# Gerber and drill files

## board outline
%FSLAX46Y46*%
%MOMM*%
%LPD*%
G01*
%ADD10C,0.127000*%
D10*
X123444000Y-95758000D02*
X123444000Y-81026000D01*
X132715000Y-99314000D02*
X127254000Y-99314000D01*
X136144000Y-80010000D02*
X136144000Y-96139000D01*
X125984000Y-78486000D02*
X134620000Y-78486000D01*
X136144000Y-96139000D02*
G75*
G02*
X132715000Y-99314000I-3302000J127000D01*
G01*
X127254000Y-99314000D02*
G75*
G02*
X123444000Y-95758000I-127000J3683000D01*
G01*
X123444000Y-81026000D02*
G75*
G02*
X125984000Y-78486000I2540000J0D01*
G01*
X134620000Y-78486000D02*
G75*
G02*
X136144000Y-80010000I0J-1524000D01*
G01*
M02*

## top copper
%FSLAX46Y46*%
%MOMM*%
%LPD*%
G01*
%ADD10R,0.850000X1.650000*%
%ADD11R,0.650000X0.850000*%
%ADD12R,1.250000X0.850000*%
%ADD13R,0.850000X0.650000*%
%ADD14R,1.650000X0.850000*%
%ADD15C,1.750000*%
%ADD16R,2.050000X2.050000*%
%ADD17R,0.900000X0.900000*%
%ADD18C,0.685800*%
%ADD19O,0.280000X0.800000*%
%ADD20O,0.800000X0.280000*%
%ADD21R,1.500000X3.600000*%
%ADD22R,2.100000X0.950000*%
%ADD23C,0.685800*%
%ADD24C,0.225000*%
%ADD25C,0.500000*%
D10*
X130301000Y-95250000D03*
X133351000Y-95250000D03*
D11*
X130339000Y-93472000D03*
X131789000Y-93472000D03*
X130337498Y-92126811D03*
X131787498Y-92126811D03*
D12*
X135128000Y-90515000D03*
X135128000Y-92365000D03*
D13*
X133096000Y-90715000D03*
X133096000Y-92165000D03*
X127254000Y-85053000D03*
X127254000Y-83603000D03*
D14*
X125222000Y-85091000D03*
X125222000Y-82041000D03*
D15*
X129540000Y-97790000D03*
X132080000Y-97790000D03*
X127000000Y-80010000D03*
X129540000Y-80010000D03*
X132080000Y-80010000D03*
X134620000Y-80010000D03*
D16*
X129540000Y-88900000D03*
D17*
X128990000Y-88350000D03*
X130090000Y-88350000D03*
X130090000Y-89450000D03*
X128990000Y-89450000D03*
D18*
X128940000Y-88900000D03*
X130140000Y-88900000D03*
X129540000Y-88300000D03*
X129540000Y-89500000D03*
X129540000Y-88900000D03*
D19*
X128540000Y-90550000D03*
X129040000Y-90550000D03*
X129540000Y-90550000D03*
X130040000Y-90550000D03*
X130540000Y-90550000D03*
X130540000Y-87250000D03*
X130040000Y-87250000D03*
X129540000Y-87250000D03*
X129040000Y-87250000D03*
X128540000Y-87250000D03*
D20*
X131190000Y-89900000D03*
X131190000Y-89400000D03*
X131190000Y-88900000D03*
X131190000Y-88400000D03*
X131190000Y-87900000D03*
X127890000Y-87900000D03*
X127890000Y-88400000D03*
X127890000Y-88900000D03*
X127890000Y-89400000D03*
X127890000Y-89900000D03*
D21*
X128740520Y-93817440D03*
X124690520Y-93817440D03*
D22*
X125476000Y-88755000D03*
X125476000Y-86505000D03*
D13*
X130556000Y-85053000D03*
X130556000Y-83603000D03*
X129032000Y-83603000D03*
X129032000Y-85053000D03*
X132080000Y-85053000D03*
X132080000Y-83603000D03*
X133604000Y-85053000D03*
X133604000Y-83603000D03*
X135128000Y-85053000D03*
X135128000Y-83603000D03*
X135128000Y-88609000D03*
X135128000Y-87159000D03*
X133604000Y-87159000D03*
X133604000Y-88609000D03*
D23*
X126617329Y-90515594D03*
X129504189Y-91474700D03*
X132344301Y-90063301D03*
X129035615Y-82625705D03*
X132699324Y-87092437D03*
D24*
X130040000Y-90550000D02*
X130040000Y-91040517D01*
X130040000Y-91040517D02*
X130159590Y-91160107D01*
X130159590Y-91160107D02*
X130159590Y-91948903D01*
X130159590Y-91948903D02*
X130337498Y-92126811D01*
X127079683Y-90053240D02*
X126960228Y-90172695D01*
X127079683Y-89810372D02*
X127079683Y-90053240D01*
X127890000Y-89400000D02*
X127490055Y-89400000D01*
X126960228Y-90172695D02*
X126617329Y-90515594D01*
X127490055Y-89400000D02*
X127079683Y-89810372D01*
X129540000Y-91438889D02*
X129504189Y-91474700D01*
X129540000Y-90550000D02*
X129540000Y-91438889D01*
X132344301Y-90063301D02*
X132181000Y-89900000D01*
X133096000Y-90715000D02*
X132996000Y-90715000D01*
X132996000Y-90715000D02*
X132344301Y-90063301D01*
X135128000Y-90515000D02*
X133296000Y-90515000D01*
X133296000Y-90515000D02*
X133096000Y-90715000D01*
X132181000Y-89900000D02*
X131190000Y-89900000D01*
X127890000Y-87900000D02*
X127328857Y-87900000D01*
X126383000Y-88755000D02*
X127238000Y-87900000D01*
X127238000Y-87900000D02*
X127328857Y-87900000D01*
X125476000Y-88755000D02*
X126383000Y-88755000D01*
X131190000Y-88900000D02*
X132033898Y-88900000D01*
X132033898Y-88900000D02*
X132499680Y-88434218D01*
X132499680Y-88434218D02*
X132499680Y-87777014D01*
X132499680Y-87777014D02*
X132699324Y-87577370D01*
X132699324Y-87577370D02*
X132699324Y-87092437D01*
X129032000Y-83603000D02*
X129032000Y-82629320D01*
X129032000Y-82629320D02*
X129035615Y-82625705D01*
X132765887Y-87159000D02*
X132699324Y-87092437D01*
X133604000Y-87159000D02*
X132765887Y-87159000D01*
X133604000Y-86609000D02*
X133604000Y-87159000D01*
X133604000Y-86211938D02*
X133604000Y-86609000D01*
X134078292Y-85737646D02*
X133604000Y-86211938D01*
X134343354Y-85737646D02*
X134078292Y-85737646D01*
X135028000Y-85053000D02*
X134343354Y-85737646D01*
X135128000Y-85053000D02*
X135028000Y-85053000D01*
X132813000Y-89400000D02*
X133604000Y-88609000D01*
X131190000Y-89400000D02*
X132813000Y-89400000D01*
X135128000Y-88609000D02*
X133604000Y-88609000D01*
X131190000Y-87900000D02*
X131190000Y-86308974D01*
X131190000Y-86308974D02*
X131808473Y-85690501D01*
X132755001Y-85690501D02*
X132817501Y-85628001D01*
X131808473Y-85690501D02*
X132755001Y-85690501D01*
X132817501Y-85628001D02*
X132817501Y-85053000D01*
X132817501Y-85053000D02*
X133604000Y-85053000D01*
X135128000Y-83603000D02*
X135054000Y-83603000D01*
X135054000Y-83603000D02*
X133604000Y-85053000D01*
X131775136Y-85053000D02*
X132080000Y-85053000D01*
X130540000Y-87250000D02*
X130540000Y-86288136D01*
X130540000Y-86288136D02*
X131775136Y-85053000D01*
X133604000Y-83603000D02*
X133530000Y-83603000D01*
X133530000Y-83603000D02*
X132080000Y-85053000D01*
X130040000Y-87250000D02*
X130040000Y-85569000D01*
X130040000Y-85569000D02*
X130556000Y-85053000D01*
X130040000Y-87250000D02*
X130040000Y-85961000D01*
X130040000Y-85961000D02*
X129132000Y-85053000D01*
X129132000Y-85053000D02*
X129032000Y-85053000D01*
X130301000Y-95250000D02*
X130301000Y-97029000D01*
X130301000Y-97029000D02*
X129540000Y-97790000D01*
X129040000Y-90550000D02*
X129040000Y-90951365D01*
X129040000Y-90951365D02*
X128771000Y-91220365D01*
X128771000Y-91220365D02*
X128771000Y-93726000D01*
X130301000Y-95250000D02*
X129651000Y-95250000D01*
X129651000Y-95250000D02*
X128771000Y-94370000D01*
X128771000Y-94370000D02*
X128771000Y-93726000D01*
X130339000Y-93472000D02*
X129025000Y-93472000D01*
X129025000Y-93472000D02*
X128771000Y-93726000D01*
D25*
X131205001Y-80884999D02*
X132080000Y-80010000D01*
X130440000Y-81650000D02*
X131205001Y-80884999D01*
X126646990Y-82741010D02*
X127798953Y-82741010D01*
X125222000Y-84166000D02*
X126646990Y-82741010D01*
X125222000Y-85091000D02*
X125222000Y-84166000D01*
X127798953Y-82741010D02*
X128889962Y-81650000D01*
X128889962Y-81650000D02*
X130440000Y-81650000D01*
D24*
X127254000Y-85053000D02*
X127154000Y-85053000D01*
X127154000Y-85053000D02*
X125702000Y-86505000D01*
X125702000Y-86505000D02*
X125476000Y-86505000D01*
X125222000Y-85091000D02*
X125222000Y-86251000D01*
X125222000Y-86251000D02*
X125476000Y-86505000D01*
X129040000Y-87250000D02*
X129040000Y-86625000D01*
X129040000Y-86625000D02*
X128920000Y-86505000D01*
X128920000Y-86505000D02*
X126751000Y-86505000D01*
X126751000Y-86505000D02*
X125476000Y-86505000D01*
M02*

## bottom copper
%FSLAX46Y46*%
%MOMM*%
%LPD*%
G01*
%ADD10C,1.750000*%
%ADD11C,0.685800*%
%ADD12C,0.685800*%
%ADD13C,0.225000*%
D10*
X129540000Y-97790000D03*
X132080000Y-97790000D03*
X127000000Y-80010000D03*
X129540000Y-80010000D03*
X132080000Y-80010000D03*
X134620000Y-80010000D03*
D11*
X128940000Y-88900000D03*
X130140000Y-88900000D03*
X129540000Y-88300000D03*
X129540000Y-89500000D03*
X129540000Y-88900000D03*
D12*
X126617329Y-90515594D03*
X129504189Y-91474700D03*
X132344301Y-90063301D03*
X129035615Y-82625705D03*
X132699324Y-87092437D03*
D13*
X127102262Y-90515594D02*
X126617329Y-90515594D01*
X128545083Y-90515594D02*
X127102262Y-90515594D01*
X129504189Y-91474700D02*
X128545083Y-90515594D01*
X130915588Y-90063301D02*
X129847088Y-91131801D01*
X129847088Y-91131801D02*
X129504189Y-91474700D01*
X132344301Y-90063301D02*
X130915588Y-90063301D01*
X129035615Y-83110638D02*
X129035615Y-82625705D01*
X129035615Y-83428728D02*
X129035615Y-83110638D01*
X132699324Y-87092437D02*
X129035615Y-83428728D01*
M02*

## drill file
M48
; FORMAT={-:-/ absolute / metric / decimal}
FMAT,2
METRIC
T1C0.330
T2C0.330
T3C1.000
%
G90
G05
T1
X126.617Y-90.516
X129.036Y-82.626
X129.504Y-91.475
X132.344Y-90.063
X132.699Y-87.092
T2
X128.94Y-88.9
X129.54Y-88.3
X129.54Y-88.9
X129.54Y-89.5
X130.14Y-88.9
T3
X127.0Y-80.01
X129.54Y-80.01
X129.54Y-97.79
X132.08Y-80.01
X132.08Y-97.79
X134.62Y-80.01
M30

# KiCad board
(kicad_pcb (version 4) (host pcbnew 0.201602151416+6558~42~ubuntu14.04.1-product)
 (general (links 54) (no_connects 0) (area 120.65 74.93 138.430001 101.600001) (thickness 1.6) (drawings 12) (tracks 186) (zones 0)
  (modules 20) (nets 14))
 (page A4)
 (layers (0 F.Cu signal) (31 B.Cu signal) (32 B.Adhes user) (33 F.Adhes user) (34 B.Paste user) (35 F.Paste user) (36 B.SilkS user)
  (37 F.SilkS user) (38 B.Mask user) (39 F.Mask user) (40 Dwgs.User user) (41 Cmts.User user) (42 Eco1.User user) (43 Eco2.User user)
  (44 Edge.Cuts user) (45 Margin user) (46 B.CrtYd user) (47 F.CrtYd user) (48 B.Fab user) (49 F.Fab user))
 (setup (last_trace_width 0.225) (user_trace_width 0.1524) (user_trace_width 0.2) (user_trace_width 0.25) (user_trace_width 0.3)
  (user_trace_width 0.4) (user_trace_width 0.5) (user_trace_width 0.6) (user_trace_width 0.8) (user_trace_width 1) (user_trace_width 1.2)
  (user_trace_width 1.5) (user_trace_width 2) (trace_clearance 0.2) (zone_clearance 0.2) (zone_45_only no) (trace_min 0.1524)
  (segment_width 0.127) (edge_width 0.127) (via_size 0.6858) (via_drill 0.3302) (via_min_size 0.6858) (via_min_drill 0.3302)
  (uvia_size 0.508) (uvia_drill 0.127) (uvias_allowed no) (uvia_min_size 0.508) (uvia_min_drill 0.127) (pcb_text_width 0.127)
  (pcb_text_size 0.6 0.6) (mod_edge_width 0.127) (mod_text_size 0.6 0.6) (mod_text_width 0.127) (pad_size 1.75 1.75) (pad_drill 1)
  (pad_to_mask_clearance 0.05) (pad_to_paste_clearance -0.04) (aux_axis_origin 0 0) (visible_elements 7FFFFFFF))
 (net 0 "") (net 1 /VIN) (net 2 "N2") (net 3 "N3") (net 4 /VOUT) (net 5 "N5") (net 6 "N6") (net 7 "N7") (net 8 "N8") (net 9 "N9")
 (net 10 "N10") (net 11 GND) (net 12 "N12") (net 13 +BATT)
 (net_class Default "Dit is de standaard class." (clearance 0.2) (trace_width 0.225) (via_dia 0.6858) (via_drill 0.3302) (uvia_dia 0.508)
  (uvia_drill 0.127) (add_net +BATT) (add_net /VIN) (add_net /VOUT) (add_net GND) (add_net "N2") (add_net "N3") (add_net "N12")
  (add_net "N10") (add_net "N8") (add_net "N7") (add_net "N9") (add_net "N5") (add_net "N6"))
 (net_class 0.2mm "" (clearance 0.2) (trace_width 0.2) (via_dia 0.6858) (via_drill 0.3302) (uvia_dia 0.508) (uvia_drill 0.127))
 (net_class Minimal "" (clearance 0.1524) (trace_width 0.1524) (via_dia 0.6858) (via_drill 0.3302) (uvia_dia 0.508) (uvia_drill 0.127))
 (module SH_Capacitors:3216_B (layer F.Cu) (at 131.826 95.25) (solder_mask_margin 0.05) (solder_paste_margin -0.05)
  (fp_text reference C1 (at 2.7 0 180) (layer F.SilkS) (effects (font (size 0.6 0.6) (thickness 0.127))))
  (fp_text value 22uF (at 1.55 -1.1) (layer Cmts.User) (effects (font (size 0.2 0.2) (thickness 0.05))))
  (pad 1 smd rect (at -1.525 0) (size 0.85 1.65) (layers F.Cu F.Paste F.Mask) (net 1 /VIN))
  (pad 2 smd rect (at 1.525 0) (size 0.85 1.65) (layers F.Cu F.Paste F.Mask)))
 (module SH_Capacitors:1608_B (layer F.Cu) (at 131.064 93.472) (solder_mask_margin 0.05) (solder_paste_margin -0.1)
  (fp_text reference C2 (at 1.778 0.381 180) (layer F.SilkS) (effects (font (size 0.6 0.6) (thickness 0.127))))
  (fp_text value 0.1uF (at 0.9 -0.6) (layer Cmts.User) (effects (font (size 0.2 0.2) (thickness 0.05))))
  (pad 1 smd rect (at -0.725 0) (size 0.65 0.85) (layers F.Cu F.Paste F.Mask) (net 1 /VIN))
  (pad 2 smd rect (at 0.725 0) (size 0.65 0.85) (layers F.Cu F.Paste F.Mask)))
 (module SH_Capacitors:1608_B (layer F.Cu) (at 131.062498 92.126811) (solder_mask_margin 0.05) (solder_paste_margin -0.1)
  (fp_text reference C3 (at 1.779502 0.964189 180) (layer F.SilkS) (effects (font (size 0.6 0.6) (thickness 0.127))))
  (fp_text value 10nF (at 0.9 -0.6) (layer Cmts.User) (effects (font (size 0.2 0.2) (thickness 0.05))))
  (pad 1 smd rect (at -0.725 0) (size 0.65 0.85) (layers F.Cu F.Paste F.Mask) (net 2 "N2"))
  (pad 2 smd rect (at 0.725 0) (size 0.65 0.85) (layers F.Cu F.Paste F.Mask)))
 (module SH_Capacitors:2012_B (layer F.Cu) (at 135.128 91.44 270) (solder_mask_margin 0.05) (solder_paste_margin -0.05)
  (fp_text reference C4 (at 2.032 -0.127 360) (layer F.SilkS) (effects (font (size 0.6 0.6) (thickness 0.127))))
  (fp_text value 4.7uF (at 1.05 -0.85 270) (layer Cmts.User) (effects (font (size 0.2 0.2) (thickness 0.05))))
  (pad 1 smd rect (at -0.925 0 270) (size 0.85 1.25) (layers F.Cu F.Paste F.Mask) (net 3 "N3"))
  (pad 2 smd rect (at 0.925 0 270) (size 0.85 1.25) (layers F.Cu F.Paste F.Mask)))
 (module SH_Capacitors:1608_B (layer F.Cu) (at 133.096 91.44 270) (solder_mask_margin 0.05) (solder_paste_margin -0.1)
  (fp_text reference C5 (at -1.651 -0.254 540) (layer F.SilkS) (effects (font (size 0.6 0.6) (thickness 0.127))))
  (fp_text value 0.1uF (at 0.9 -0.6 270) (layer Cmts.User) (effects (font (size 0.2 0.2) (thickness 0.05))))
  (pad 1 smd rect (at -0.725 0 270) (size 0.65 0.85) (layers F.Cu F.Paste F.Mask) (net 3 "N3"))
  (pad 2 smd rect (at 0.725 0 270) (size 0.65 0.85) (layers F.Cu F.Paste F.Mask)))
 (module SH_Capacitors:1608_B (layer F.Cu) (at 127.254 84.328 90) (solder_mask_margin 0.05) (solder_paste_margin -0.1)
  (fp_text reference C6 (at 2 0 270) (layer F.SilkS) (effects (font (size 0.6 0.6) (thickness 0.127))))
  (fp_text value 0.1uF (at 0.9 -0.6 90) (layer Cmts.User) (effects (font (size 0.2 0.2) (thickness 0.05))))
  (pad 1 smd rect (at -0.725 0 90) (size 0.65 0.85) (layers F.Cu F.Paste F.Mask) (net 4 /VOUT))
  (pad 2 smd rect (at 0.725 0 90) (size 0.65 0.85) (layers F.Cu F.Paste F.Mask)))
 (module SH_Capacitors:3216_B (layer F.Cu) (at 125.222 83.566 90) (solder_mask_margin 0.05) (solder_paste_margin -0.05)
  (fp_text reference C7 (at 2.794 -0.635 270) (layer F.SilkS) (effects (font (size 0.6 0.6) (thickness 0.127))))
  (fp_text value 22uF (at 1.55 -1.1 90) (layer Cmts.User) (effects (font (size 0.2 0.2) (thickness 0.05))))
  (pad 1 smd rect (at -1.525 0 90) (size 0.85 1.65) (layers F.Cu F.Paste F.Mask) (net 4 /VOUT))
  (pad 2 smd rect (at 1.525 0 90) (size 0.85 1.65) (layers F.Cu F.Paste F.Mask)))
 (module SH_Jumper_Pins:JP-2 (layer F.Cu) (at 130.81 97.79)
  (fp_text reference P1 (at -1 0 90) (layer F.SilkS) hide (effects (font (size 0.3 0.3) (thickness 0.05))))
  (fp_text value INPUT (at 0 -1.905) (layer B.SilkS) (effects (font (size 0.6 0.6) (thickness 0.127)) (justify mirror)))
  (pad 1 thru_hole circle (at -1.27 0) (size 1.75 1.75) (drill 1) (layers *.Cu *.Mask) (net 1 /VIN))
  (pad 2 thru_hole circle (at 1.27 0) (size 1.75 1.75) (drill 1) (layers *.Cu *.Mask)))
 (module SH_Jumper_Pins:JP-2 (layer F.Cu) (at 128.27 80.01)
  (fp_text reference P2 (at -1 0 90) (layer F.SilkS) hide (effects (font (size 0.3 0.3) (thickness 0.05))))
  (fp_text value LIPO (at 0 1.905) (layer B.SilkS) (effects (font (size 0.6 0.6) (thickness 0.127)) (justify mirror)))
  (pad 1 thru_hole circle (at -1.27 0) (size 1.75 1.75) (drill 1) (layers *.Cu *.Mask))
  (pad 2 thru_hole circle (at 1.27 0) (size 1.75 1.75) (drill 1) (layers *.Cu *.Mask)))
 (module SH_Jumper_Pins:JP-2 (layer F.Cu) (at 133.35 80.01)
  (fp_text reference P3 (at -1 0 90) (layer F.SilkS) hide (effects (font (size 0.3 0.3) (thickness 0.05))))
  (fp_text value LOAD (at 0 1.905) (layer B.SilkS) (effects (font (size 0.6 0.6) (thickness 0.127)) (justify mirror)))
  (pad 1 thru_hole circle (at -1.27 0) (size 1.75 1.75) (drill 1) (layers *.Cu *.Mask) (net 4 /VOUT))
  (pad 2 thru_hole circle (at 1.27 0) (size 1.75 1.75) (drill 1) (layers *.Cu *.Mask)))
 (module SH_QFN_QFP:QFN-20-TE (layer F.Cu) (at 129.54 88.9) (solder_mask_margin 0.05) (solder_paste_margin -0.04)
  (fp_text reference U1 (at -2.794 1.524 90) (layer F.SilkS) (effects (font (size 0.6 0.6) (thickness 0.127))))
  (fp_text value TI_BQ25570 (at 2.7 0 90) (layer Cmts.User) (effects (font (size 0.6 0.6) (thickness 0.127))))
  (pad 21 smd rect (at 0 0) (size 2.05 2.05) (layers F.Cu F.Mask) (zone_connect 2))
  (pad 21 smd rect (at -0.55 -0.55) (size 0.9 0.9) (layers F.Cu F.Paste F.Mask))
  (pad 21 smd rect (at 0.55 -0.55) (size 0.9 0.9) (layers F.Cu F.Paste F.Mask))
  (pad 21 smd rect (at 0.55 0.55) (size 0.9 0.9) (layers F.Cu F.Paste F.Mask))
  (pad 21 smd rect (at -0.55 0.55) (size 0.9 0.9) (layers F.Cu F.Paste F.Mask))
  (pad 21 thru_hole circle (at -0.6 0) (size 0.6858 0.6858) (drill 0.3302) (layers *.Cu))
  (pad 21 thru_hole circle (at 0.6 0) (size 0.6858 0.6858) (drill 0.3302) (layers *.Cu))
  (pad 21 thru_hole circle (at 0 -0.6) (size 0.6858 0.6858) (drill 0.3302) (layers *.Cu))
  (pad 21 thru_hole circle (at 0 0.6) (size 0.6858 0.6858) (drill 0.3302) (layers *.Cu))
  (pad 21 thru_hole circle (at 0 0) (size 0.6858 0.6858) (drill 0.3302) (layers *.Cu))
  (pad 1 smd oval (at -1 1.65) (size 0.28 0.8) (layers F.Cu F.Paste F.Mask))
  (pad 2 smd oval (at -0.5 1.65) (size 0.28 0.8) (layers F.Cu F.Paste F.Mask) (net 1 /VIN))
  (pad 3 smd oval (at 0 1.65) (size 0.28 0.8) (layers F.Cu F.Paste F.Mask) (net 3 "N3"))
  (pad 4 smd oval (at 0.5 1.65) (size 0.28 0.8) (layers F.Cu F.Paste F.Mask) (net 2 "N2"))
  (pad 5 smd oval (at 1 1.65) (size 0.28 0.8) (layers F.Cu F.Paste F.Mask))
  (pad 11 smd oval (at 1 -1.65) (size 0.28 0.8) (layers F.Cu F.Paste F.Mask) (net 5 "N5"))
  (pad 12 smd oval (at 0.5 -1.65) (size 0.28 0.8) (layers F.Cu F.Paste F.Mask) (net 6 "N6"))
  (pad 13 smd oval (at 0 -1.65) (size 0.28 0.8) (layers F.Cu F.Paste F.Mask))
  (pad 14 smd oval (at -0.5 -1.65) (size 0.28 0.8) (layers F.Cu F.Paste F.Mask) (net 4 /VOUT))
  (pad 15 smd oval (at -1 -1.65) (size 0.28 0.8) (layers F.Cu F.Paste F.Mask))
  (pad 6 smd oval (at 1.65 1 90) (size 0.28 0.8) (layers F.Cu F.Paste F.Mask) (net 3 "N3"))
  (pad 7 smd oval (at 1.65 0.5 90) (size 0.28 0.8) (layers F.Cu F.Paste F.Mask) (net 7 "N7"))
  (pad 8 smd oval (at 1.65 0 90) (size 0.28 0.8) (layers F.Cu F.Paste F.Mask) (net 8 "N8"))
  (pad 9 smd oval (at 1.65 -0.5 90) (size 0.28 0.8) (layers F.Cu F.Paste F.Mask))
  (pad 10 smd oval (at 1.65 -1 90) (size 0.28 0.8) (layers F.Cu F.Paste F.Mask) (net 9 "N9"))
  (pad 16 smd oval (at -1.65 -1 90) (size 0.28 0.8) (layers F.Cu F.Paste F.Mask) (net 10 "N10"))
  (pad 17 smd oval (at -1.65 -0.5 90) (size 0.28 0.8) (layers F.Cu F.Paste F.Mask))
  (pad 18 smd oval (at -1.65 0 90) (size 0.28 0.8) (layers F.Cu F.Paste F.Mask))
  (pad 19 smd oval (at -1.65 0.5 90) (size 0.28 0.8) (layers F.Cu F.Paste F.Mask) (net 3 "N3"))
  (pad 20 smd oval (at -1.65 1 90) (size 0.28 0.8) (layers F.Cu F.Paste F.Mask)))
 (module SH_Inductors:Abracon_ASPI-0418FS (layer F.Cu) (at 126.71552 93.81744 180) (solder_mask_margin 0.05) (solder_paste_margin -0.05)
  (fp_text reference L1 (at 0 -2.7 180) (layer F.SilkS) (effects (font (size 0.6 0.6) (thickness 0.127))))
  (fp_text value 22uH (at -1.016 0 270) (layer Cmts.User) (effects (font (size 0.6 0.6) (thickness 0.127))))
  (pad 1 smd rect (at -2.025 0 180) (size 1.5 3.6) (layers F.Cu F.Paste F.Mask) (zone_connect 2))
  (pad 2 smd rect (at 2.025 0 180) (size 1.5 3.6) (layers F.Cu F.Paste F.Mask) (zone_connect 2)))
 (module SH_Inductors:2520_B (layer F.Cu) (at 125.476 87.63 90) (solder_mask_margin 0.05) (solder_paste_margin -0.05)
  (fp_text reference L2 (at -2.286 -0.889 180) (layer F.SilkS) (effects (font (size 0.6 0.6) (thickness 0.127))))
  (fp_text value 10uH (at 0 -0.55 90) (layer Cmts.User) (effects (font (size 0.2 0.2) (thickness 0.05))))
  (pad 1 smd rect (at -1.125 0 90) (size 0.95 2.1) (layers F.Cu F.Paste F.Mask) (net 10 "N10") (zone_connect 2))
  (pad 2 smd rect (at 1.125 0 90) (size 0.95 2.1) (layers F.Cu F.Paste F.Mask) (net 4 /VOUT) (zone_connect 2)))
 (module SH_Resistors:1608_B (layer F.Cu) (at 130.556 84.328 90) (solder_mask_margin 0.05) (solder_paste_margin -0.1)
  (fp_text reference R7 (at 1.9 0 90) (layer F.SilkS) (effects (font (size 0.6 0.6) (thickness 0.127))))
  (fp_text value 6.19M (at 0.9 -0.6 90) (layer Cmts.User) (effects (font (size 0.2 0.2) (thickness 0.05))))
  (pad 1 smd rect (at -0.725 0 90) (size 0.65 0.85) (layers F.Cu F.Paste F.Mask) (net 6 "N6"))
  (pad 2 smd rect (at 0.725 0 90) (size 0.65 0.85) (layers F.Cu F.Paste F.Mask)))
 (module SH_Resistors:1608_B (layer F.Cu) (at 129.032 84.328 270) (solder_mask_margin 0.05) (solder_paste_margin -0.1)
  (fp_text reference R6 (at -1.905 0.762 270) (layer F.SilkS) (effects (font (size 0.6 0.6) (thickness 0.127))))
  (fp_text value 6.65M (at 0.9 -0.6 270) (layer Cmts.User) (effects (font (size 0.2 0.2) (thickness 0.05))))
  (pad 1 smd rect (at -0.725 0 270) (size 0.65 0.85) (layers F.Cu F.Paste F.Mask) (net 8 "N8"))
  (pad 2 smd rect (at 0.725 0 270) (size 0.65 0.85) (layers F.Cu F.Paste F.Mask) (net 6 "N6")))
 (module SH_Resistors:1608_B (layer F.Cu) (at 132.08 84.328 90) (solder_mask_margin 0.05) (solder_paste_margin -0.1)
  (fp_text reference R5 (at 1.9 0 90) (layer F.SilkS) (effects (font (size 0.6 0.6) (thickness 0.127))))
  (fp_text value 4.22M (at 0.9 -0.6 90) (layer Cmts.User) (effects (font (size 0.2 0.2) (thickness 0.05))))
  (pad 1 smd rect (at -0.725 0 90) (size 0.65 0.85) (layers F.Cu F.Paste F.Mask) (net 5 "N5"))
  (pad 2 smd rect (at 0.725 0 90) (size 0.65 0.85) (layers F.Cu F.Paste F.Mask)))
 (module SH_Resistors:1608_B (layer F.Cu) (at 133.604 84.328 90) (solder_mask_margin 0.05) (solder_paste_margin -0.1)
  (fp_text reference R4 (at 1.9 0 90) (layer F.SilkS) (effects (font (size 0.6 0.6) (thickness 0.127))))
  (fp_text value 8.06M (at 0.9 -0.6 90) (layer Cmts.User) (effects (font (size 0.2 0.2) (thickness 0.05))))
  (pad 1 smd rect (at -0.725 0 90) (size 0.65 0.85) (layers F.Cu F.Paste F.Mask) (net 9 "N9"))
  (pad 2 smd rect (at 0.725 0 90) (size 0.65 0.85) (layers F.Cu F.Paste F.Mask) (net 5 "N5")))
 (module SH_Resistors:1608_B (layer F.Cu) (at 135.128 84.328 90) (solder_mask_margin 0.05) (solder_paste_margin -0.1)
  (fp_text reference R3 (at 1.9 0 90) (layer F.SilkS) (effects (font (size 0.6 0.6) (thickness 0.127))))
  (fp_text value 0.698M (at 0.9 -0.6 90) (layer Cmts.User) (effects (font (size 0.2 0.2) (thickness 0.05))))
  (pad 1 smd rect (at -0.725 0 90) (size 0.65 0.85) (layers F.Cu F.Paste F.Mask) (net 8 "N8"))
  (pad 2 smd rect (at 0.725 0 90) (size 0.65 0.85) (layers F.Cu F.Paste F.Mask) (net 9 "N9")))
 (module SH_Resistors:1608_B (layer F.Cu) (at 135.128 87.884 90) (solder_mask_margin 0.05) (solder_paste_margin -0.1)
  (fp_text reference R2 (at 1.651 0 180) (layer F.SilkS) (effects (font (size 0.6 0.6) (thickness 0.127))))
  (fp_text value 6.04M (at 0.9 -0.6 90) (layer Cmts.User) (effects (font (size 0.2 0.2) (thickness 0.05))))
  (pad 1 smd rect (at -0.725 0 90) (size 0.65 0.85) (layers F.Cu F.Paste F.Mask) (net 7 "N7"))
  (pad 2 smd rect (at 0.725 0 90) (size 0.65 0.85) (layers F.Cu F.Paste F.Mask)))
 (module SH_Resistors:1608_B (layer F.Cu) (at 133.604 87.884 270) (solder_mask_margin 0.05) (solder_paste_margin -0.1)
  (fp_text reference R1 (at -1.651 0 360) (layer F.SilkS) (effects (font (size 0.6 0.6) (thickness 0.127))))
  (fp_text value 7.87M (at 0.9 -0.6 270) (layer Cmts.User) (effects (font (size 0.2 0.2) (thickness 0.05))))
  (pad 1 smd rect (at -0.725 0 270) (size 0.65 0.85) (layers F.Cu F.Paste F.Mask) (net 8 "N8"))
  (pad 2 smd rect (at 0.725 0 270) (size 0.65 0.85) (layers F.Cu F.Paste F.Mask) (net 7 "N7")))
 (gr_line (start 123.444 95.758) (end 123.444 81.026) (angle 90) (layer Edge.Cuts) (width 0.127))
 (gr_line (start 132.715 99.314) (end 127.254 99.314) (angle 90) (layer Edge.Cuts) (width 0.127))
 (gr_line (start 136.144 80.01) (end 136.144 96.139) (angle 90) (layer Edge.Cuts) (width 0.127))
 (gr_line (start 125.984 78.486) (end 134.62 78.486) (angle 90) (layer Edge.Cuts) (width 0.127))
 (gr_arc (start 132.842 96.012) (end 136.144 96.139) (angle 90) (layer Edge.Cuts) (width 0.127))
 (gr_arc (start 127.127 95.631) (end 127.254 99.314) (angle 90) (layer Edge.Cuts) (width 0.127))
 (gr_arc (start 125.984 81.026) (end 123.444 81.026) (angle 90) (layer Edge.Cuts) (width 0.127))
 (gr_arc (start 134.62 80.01) (end 134.62 78.486) (angle 90) (layer Edge.Cuts) (width 0.127))
 (segment (start 130.04 90.55) (end 130.04 91.040517) (width 0.225) (layer F.Cu) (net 2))
 (segment (start 130.04 91.040517) (end 130.15959 91.160107) (width 0.225) (layer F.Cu) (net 2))
 (segment (start 130.15959 91.160107) (end 130.15959 91.948903) (width 0.225) (layer F.Cu) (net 2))
 (segment (start 130.15959 91.948903) (end 130.337498 92.126811) (width 0.225) (layer F.Cu) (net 2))
 (segment (start 127.079683 90.05324) (end 126.960228 90.172695) (width 0.225) (layer F.Cu) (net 3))
 (segment (start 127.079683 89.810372) (end 127.079683 90.05324) (width 0.225) (layer F.Cu) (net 3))
 (segment (start 127.89 89.4) (end 127.490055 89.4) (width 0.225) (layer F.Cu) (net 3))
 (segment (start 127.102262 90.515594) (end 126.617329 90.515594) (width 0.225) (layer B.Cu) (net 3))
 (segment (start 128.545083 90.515594) (end 127.102262 90.515594) (width 0.225) (layer B.Cu) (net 3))
 (segment (start 126.960228 90.172695) (end 126.617329 90.515594) (width 0.225) (layer F.Cu) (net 3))
 (segment (start 129.504189 91.4747) (end 128.545083 90.515594) (width 0.225) (layer B.Cu) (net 3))
 (segment (start 127.490055 89.4) (end 127.079683 89.810372) (width 0.225) (layer F.Cu) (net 3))
 (segment (start 130.915588 90.063301) (end 129.847088 91.131801) (width 0.225) (layer B.Cu) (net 3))
 (segment (start 129.847088 91.131801) (end 129.504189 91.4747) (width 0.225) (layer B.Cu) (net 3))
 (segment (start 132.344301 90.063301) (end 130.915588 90.063301) (width 0.225) (layer B.Cu) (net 3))
 (segment (start 129.54 91.438889) (end 129.504189 91.4747) (width 0.225) (layer F.Cu) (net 3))
 (segment (start 129.54 90.55) (end 129.54 91.438889) (width 0.225) (layer F.Cu) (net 3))
 (segment (start 132.344301 90.063301) (end 132.181 89.9) (width 0.225) (layer F.Cu) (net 3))
 (segment (start 133.096 90.715) (end 132.996 90.715) (width 0.225) (layer F.Cu) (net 3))
 (segment (start 132.996 90.715) (end 132.344301 90.063301) (width 0.225) (layer F.Cu) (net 3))
 (segment (start 135.128 90.515) (end 133.296 90.515) (width 0.225) (layer F.Cu) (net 3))
 (segment (start 133.296 90.515) (end 133.096 90.715) (width 0.225) (layer F.Cu) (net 3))
 (segment (start 132.181 89.9) (end 131.19 89.9) (width 0.225) (layer F.Cu) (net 3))
 (segment (start 127.89 87.9) (end 127.328857 87.9) (width 0.225) (layer F.Cu) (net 10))
 (segment (start 126.383 88.755) (end 127.238 87.9) (width 0.225) (layer F.Cu) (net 10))
 (segment (start 127.238 87.9) (end 127.328857 87.9) (width 0.225) (layer F.Cu) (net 10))
 (segment (start 125.476 88.755) (end 126.383 88.755) (width 0.225) (layer F.Cu) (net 10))
 (segment (start 131.19 88.9) (end 132.033898 88.9) (width 0.225) (layer F.Cu) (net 8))
 (segment (start 132.033898 88.9) (end 132.49968 88.434218) (width 0.225) (layer F.Cu) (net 8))
 (segment (start 132.49968 88.434218) (end 132.49968 87.777014) (width 0.225) (layer F.Cu) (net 8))
 (segment (start 132.49968 87.777014) (end 132.699324 87.57737) (width 0.225) (layer F.Cu) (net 8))
 (segment (start 132.699324 87.57737) (end 132.699324 87.092437) (width 0.225) (layer F.Cu) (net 8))
 (segment (start 129.035615 83.110638) (end 129.035615 82.625705) (width 0.225) (layer B.Cu) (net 8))
 (segment (start 129.035615 83.428728) (end 129.035615 83.110638) (width 0.225) (layer B.Cu) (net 8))
 (segment (start 132.699324 87.092437) (end 129.035615 83.428728) (width 0.225) (layer B.Cu) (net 8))
 (segment (start 129.032 83.603) (end 129.032 82.62932) (width 0.225) (layer F.Cu) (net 8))
 (segment (start 129.032 82.62932) (end 129.035615 82.625705) (width 0.225) (layer F.Cu) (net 8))
 (segment (start 132.765887 87.159) (end 132.699324 87.092437) (width 0.225) (layer F.Cu) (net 8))
 (segment (start 133.604 87.159) (end 132.765887 87.159) (width 0.225) (layer F.Cu) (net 8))
 (segment (start 133.604 86.609) (end 133.604 87.159) (width 0.225) (layer F.Cu) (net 8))
 (segment (start 133.604 86.211938) (end 133.604 86.609) (width 0.225) (layer F.Cu) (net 8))
 (segment (start 134.078292 85.737646) (end 133.604 86.211938) (width 0.225) (layer F.Cu) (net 8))
 (segment (start 134.343354 85.737646) (end 134.078292 85.737646) (width 0.225) (layer F.Cu) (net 8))
 (segment (start 135.028 85.053) (end 134.343354 85.737646) (width 0.225) (layer F.Cu) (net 8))
 (segment (start 135.128 85.053) (end 135.028 85.053) (width 0.225) (layer F.Cu) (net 8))
 (segment (start 132.813 89.4) (end 133.604 88.609) (width 0.225) (layer F.Cu) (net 7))
 (segment (start 131.19 89.4) (end 132.813 89.4) (width 0.225) (layer F.Cu) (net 7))
 (segment (start 135.128 88.609) (end 133.604 88.609) (width 0.225) (layer F.Cu) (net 7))
 (segment (start 131.19 87.9) (end 131.19 86.308974) (width 0.225) (layer F.Cu) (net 9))
 (segment (start 131.19 86.308974) (end 131.808473 85.690501) (width 0.225) (layer F.Cu) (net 9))
 (segment (start 132.755001 85.690501) (end 132.817501 85.628001) (width 0.225) (layer F.Cu) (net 9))
 (segment (start 131.808473 85.690501) (end 132.755001 85.690501) (width 0.225) (layer F.Cu) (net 9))
 (segment (start 132.817501 85.628001) (end 132.817501 85.053) (width 0.225) (layer F.Cu) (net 9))
 (segment (start 132.817501 85.053) (end 133.604 85.053) (width 0.225) (layer F.Cu) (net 9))
 (segment (start 135.128 83.603) (end 135.054 83.603) (width 0.225) (layer F.Cu) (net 9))
 (segment (start 135.054 83.603) (end 133.604 85.053) (width 0.225) (layer F.Cu) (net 9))
 (segment (start 131.775136 85.053) (end 132.08 85.053) (width 0.225) (layer F.Cu) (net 5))
 (segment (start 130.54 87.25) (end 130.54 86.288136) (width 0.225) (layer F.Cu) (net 5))
 (segment (start 130.54 86.288136) (end 131.775136 85.053) (width 0.225) (layer F.Cu) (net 5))
 (segment (start 133.604 83.603) (end 133.53 83.603) (width 0.225) (layer F.Cu) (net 5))
 (segment (start 133.53 83.603) (end 132.08 85.053) (width 0.225) (layer F.Cu) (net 5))
 (segment (start 130.04 87.25) (end 130.04 85.569) (width 0.225) (layer F.Cu) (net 6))
 (segment (start 130.04 85.569) (end 130.556 85.053) (width 0.225) (layer F.Cu) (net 6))
 (segment (start 130.04 87.25) (end 130.04 85.961) (width 0.225) (layer F.Cu) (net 6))
 (segment (start 130.04 85.961) (end 129.132 85.053) (width 0.225) (layer F.Cu) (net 6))
 (segment (start 129.132 85.053) (end 129.032 85.053) (width 0.225) (layer F.Cu) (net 6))
 (segment (start 130.301 95.25) (end 130.301 97.029) (width 0.225) (layer F.Cu) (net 1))
 (segment (start 130.301 97.029) (end 129.54 97.79) (width 0.225) (layer F.Cu) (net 1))
 (segment (start 129.04 90.55) (end 129.04 90.951365) (width 0.225) (layer F.Cu) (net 1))
 (segment (start 129.04 90.951365) (end 128.771 91.220365) (width 0.225) (layer F.Cu) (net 1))
 (segment (start 128.771 91.220365) (end 128.771 93.726) (width 0.225) (layer F.Cu) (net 1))
 (segment (start 130.301 95.25) (end 129.651 95.25) (width 0.225) (layer F.Cu) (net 1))
 (segment (start 129.651 95.25) (end 128.771 94.37) (width 0.225) (layer F.Cu) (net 1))
 (segment (start 128.771 94.37) (end 128.771 93.726) (width 0.225) (layer F.Cu) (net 1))
 (segment (start 130.339 93.472) (end 129.025 93.472) (width 0.225) (layer F.Cu) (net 1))
 (segment (start 129.025 93.472) (end 128.771 93.726) (width 0.225) (layer F.Cu) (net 1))
 (segment (start 131.205001 80.884999) (end 132.08 80.01) (width 0.5) (layer F.Cu) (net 4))
 (segment (start 130.44 81.65) (end 131.205001 80.884999) (width 0.5) (layer F.Cu) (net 4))
 (segment (start 126.64699 82.74101) (end 127.798953 82.74101) (width 0.5) (layer F.Cu) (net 4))
 (segment (start 125.222 84.166) (end 126.64699 82.74101) (width 0.5) (layer F.Cu) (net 4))
 (segment (start 125.222 85.091) (end 125.222 84.166) (width 0.5) (layer F.Cu) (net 4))
 (segment (start 127.798953 82.74101) (end 128.889962 81.65) (width 0.5) (layer F.Cu) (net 4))
 (segment (start 128.889962 81.65) (end 130.44 81.65) (width 0.5) (layer F.Cu) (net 4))
 (segment (start 127.254 85.053) (end 127.154 85.053) (width 0.225) (layer F.Cu) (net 4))
 (segment (start 127.154 85.053) (end 125.702 86.505) (width 0.225) (layer F.Cu) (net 4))
 (segment (start 125.702 86.505) (end 125.476 86.505) (width 0.225) (layer F.Cu) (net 4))
 (segment (start 125.222 85.091) (end 125.222 86.251) (width 0.225) (layer F.Cu) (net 4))
 (segment (start 125.222 86.251) (end 125.476 86.505) (width 0.225) (layer F.Cu) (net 4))
 (segment (start 129.04 87.25) (end 129.04 86.625) (width 0.225) (layer F.Cu) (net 4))
 (segment (start 129.04 86.625) (end 128.92 86.505) (width 0.225) (layer F.Cu) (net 4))
 (segment (start 128.92 86.505) (end 126.751 86.505) (width 0.225) (layer F.Cu) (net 4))
 (segment (start 126.751 86.505) (end 125.476 86.505) (width 0.225) (layer F.Cu) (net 4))
 (via (at 126.617329 90.515594) (size 0.6858) (layers F.Cu B.Cu) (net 3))
 (via (at 129.504189 91.4747) (size 0.6858) (layers F.Cu B.Cu) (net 3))
 (via (at 132.344301 90.063301) (size 0.6858) (layers F.Cu B.Cu) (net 3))
 (via (at 129.035615 82.625705) (size 0.6858) (layers F.Cu B.Cu) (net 8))
 (via (at 132.699324 87.092437) (size 0.6858) (layers F.Cu B.Cu) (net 8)))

